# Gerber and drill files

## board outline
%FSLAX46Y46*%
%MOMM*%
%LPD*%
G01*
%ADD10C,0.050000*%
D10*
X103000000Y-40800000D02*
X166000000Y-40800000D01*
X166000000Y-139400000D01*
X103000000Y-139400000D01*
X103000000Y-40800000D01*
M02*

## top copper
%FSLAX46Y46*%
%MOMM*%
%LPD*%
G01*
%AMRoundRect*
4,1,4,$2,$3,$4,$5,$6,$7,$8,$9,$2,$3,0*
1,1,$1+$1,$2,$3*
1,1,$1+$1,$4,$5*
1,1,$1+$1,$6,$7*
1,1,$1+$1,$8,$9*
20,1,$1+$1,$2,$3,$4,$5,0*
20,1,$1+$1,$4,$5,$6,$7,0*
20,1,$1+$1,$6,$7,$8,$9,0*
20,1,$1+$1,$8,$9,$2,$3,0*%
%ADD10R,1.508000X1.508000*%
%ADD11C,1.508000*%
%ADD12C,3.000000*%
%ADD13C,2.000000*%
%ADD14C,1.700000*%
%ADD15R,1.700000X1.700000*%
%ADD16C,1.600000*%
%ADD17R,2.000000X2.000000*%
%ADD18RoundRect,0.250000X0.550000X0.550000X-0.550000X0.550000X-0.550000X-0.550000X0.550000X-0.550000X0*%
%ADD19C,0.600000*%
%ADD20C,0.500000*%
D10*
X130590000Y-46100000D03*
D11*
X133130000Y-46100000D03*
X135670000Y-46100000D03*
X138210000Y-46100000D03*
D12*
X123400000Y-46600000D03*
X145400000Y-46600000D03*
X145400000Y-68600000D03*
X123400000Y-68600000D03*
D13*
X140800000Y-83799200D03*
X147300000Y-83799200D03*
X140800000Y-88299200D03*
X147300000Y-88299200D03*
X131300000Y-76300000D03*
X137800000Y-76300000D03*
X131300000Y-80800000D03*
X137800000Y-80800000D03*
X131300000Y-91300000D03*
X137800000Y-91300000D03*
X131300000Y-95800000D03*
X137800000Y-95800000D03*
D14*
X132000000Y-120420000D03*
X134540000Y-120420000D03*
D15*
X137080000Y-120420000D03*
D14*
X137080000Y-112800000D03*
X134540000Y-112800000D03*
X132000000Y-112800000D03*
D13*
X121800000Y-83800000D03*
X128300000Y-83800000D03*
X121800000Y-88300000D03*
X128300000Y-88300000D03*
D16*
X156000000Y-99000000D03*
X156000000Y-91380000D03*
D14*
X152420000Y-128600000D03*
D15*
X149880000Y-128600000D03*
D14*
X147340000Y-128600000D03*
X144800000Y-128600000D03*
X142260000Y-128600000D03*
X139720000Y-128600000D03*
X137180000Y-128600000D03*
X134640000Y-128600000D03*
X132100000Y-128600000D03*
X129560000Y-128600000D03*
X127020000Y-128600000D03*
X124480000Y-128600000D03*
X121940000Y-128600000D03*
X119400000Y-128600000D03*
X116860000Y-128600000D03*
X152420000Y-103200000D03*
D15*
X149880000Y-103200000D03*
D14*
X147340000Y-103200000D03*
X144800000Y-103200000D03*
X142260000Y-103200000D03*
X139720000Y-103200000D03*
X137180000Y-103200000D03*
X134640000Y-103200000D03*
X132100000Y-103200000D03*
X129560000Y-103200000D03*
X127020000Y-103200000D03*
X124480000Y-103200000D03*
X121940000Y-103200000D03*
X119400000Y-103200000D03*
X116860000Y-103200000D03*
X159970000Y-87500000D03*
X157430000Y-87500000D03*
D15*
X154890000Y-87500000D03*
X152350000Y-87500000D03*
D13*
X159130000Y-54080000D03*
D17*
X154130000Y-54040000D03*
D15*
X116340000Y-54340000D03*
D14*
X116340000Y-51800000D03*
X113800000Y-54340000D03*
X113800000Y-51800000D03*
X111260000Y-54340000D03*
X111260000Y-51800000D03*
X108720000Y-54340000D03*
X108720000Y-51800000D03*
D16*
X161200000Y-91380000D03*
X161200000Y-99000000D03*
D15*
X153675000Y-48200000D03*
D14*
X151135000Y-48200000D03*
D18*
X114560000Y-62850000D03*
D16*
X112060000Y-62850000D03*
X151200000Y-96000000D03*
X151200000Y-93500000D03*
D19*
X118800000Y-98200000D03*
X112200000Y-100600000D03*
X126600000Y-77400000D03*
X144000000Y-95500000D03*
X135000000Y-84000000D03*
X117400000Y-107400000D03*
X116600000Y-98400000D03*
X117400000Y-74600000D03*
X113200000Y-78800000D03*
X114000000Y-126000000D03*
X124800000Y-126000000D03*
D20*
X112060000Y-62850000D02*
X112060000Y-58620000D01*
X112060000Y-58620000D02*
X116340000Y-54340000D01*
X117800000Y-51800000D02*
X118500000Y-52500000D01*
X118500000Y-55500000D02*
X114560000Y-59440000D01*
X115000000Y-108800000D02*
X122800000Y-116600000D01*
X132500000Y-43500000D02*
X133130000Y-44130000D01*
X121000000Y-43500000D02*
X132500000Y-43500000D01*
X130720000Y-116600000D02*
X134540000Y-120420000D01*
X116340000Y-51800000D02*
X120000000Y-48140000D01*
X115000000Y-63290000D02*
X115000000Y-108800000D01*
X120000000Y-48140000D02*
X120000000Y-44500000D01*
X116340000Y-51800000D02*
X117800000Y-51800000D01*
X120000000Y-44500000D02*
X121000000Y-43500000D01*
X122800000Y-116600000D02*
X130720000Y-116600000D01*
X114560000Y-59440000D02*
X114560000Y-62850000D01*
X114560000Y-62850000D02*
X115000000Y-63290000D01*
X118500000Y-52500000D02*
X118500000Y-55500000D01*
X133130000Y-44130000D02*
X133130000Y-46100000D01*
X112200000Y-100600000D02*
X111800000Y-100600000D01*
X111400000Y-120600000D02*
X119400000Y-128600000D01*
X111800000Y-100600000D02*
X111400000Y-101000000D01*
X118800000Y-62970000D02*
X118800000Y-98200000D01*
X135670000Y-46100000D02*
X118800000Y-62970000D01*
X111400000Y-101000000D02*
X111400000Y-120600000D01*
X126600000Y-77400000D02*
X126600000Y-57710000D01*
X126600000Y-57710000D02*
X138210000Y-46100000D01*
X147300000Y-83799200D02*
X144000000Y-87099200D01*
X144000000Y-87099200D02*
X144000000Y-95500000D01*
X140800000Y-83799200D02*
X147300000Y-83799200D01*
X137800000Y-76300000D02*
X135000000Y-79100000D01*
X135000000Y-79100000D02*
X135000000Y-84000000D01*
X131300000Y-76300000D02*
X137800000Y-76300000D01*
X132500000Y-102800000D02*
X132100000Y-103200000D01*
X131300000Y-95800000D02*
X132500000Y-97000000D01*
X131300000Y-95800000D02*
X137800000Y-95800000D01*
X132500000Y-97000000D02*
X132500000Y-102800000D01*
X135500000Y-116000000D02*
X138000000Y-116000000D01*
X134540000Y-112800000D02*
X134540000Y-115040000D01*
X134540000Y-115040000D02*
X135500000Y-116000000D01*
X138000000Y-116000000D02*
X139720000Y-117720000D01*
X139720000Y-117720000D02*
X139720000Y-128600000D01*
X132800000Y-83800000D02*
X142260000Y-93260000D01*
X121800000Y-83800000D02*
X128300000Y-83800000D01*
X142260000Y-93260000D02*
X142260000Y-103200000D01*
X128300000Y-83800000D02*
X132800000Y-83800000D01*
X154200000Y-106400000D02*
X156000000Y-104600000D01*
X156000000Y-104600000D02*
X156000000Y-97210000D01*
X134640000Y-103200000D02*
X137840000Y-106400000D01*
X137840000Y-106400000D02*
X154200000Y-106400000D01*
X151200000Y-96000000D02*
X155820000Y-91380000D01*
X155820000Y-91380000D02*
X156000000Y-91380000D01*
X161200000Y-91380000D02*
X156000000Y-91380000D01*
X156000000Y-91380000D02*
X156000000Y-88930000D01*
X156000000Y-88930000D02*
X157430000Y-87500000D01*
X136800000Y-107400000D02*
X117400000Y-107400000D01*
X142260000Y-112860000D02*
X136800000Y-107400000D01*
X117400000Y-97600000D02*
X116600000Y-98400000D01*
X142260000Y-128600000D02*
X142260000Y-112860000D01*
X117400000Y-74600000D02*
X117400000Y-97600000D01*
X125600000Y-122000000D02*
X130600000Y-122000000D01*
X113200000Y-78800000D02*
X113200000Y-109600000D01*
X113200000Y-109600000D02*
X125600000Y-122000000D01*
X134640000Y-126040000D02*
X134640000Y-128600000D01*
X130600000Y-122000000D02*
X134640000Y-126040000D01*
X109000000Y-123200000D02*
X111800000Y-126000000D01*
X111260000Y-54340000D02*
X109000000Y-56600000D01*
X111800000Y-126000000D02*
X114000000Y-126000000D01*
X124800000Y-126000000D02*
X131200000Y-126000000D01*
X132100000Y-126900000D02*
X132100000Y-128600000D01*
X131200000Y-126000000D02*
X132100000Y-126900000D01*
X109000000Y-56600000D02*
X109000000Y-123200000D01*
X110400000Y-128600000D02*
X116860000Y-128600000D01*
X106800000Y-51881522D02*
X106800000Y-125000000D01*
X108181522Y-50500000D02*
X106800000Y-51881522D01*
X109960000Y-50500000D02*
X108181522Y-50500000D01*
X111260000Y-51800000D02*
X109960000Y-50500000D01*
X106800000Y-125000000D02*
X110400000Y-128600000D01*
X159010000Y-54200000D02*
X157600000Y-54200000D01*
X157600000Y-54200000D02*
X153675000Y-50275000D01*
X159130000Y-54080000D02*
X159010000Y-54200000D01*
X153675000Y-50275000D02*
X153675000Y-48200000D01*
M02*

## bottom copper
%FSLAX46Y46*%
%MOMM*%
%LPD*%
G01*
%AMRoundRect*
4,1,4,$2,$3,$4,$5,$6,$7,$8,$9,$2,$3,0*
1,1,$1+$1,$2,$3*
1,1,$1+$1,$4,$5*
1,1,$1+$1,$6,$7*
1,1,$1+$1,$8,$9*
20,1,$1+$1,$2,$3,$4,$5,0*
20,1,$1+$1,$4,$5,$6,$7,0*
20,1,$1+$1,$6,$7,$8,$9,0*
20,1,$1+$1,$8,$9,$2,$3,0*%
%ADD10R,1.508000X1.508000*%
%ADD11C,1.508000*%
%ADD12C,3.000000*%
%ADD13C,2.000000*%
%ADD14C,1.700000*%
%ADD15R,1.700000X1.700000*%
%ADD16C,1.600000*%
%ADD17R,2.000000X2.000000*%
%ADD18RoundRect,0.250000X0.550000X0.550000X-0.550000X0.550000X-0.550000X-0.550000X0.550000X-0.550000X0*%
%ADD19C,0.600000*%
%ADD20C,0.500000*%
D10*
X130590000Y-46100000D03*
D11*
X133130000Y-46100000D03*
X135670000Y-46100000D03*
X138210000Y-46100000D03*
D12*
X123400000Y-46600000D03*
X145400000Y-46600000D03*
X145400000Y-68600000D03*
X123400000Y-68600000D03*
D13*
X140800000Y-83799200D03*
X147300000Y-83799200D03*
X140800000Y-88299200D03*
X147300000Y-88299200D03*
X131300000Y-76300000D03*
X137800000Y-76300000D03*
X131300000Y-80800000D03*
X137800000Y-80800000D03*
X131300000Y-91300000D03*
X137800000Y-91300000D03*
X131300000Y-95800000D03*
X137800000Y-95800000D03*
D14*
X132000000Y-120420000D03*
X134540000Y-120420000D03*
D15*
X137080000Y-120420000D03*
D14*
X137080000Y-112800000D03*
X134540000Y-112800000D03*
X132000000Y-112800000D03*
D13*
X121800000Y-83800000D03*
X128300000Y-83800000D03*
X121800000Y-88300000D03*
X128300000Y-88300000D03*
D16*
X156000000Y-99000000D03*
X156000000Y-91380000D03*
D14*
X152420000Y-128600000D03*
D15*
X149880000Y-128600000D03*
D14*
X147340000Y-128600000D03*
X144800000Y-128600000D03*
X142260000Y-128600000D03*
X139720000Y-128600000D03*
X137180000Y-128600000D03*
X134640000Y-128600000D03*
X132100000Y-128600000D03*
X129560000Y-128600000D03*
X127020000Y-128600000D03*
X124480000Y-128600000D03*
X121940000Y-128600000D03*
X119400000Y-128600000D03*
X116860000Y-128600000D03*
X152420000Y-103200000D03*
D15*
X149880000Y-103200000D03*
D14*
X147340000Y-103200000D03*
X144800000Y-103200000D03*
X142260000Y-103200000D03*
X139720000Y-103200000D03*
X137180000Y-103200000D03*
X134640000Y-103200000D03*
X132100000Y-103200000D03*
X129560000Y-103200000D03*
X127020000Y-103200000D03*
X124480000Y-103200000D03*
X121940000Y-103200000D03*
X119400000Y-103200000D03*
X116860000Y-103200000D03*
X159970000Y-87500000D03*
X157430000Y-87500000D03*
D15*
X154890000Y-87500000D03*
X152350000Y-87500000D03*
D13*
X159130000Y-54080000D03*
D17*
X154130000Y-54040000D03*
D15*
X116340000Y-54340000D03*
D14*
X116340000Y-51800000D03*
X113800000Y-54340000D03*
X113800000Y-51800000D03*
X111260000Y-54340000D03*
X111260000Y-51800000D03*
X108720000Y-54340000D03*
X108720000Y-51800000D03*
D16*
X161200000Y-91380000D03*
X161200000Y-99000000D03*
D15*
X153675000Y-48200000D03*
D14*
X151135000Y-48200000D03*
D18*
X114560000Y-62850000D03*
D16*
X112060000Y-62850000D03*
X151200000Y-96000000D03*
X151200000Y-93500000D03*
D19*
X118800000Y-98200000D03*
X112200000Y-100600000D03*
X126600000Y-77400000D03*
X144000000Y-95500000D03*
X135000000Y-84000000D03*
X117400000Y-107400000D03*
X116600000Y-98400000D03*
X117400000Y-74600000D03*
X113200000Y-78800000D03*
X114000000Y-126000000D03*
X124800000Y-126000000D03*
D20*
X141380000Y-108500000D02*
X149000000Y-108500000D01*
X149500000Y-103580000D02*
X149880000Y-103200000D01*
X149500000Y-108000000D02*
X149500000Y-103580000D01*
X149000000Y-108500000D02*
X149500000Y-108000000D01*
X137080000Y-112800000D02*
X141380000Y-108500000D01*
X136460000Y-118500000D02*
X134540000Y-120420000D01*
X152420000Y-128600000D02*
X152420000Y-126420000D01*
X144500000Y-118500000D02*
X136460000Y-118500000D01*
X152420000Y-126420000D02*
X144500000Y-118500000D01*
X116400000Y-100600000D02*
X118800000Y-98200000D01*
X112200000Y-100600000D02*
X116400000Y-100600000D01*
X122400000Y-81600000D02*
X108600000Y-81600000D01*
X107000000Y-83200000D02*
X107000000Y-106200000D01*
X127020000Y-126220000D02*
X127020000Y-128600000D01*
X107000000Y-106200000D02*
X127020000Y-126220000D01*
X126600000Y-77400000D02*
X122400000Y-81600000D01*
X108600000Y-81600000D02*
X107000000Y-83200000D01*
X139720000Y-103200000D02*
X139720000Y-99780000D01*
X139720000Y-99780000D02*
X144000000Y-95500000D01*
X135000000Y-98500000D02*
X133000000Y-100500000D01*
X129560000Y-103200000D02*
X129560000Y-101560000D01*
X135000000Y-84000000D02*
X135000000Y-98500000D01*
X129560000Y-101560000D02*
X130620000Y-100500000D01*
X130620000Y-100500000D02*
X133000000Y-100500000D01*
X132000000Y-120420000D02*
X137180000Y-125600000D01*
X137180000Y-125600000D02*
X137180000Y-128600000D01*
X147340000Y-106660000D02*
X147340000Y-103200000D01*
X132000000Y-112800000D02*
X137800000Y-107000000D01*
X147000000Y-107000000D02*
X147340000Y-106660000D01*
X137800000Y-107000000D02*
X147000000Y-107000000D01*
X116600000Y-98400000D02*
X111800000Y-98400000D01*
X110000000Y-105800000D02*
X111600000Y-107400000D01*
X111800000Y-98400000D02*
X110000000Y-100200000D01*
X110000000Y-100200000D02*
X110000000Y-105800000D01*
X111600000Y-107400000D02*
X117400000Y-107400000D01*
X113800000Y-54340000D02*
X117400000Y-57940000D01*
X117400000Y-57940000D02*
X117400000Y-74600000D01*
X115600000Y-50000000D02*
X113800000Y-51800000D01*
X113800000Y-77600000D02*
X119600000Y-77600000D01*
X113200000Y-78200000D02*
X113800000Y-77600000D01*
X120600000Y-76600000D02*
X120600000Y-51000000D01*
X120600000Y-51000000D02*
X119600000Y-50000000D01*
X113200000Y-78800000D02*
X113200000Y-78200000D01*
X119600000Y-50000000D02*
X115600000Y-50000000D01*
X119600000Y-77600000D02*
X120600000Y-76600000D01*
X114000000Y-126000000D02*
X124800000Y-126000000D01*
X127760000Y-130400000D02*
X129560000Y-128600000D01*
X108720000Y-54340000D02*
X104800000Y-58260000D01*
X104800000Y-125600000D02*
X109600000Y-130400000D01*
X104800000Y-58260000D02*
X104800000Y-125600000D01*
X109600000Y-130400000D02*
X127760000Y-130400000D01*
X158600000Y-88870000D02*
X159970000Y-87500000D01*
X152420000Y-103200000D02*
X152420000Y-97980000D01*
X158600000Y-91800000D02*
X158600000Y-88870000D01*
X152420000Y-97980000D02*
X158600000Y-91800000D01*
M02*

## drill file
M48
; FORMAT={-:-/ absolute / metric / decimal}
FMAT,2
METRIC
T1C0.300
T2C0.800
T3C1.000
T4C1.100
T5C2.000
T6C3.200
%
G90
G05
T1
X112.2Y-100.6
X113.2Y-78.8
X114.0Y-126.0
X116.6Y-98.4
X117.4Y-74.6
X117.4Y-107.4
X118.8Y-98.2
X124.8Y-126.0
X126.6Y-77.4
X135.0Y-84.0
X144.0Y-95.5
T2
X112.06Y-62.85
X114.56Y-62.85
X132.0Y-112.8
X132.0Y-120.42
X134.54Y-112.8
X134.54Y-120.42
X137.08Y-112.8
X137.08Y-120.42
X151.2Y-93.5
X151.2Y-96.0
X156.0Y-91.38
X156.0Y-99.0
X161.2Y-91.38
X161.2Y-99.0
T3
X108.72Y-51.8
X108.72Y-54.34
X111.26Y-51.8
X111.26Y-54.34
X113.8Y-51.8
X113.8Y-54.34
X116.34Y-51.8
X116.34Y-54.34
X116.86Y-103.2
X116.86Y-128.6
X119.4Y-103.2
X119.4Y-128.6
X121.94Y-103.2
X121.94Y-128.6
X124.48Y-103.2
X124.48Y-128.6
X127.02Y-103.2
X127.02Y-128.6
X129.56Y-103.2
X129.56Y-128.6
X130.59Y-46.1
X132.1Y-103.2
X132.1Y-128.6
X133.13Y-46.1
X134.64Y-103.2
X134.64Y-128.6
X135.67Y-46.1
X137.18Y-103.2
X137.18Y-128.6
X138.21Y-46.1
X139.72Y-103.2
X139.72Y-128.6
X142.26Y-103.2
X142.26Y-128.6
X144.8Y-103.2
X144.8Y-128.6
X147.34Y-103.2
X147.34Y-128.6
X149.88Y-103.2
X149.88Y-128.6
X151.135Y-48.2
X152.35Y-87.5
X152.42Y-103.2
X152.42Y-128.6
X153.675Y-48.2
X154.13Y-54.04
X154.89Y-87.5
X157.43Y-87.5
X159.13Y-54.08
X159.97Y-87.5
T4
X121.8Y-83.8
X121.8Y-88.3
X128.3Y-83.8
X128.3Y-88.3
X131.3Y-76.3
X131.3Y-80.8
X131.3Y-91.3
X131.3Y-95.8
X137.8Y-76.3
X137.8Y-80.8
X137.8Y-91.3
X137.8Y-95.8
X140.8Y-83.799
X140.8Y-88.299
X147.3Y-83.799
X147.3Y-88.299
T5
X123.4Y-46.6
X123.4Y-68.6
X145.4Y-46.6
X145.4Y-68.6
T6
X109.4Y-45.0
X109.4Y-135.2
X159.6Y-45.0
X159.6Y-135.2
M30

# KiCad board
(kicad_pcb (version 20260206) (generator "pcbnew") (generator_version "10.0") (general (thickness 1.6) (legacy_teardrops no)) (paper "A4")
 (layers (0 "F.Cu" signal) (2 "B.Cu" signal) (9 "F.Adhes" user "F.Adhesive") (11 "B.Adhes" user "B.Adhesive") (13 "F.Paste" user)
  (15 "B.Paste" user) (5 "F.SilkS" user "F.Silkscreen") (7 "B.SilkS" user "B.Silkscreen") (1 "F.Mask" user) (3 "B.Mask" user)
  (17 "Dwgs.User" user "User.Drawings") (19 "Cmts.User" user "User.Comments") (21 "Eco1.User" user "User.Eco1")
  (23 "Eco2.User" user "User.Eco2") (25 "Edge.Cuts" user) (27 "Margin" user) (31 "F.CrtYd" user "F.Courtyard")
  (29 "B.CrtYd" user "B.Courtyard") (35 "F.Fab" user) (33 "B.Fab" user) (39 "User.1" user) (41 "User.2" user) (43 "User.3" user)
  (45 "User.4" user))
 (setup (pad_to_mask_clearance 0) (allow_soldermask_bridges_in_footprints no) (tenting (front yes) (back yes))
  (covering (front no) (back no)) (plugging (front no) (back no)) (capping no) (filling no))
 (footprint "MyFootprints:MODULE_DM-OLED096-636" (layer "F.Cu") (at 134.4 57.6)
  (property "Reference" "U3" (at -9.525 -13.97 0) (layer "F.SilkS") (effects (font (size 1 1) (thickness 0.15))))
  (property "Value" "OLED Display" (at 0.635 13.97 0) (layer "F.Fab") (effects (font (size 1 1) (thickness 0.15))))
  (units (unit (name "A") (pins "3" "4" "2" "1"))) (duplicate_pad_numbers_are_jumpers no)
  (pad "1" thru_hole rect (at -3.81 -11.5) (size 1.508 1.508) (drill 1) (layers "*.Cu" "*.Mask") (remove_unused_layers no) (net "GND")
   (solder_mask_margin 0.102))
  (pad "2" thru_hole circle (at -1.27 -11.5) (size 1.508 1.508) (drill 1) (layers "*.Cu" "*.Mask") (remove_unused_layers no) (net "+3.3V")
   (solder_mask_margin 0.102))
  (pad "3" thru_hole circle (at 1.27 -11.5) (size 1.508 1.508) (drill 1) (layers "*.Cu" "*.Mask") (remove_unused_layers no) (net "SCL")
   (solder_mask_margin 0.102))
  (pad "4" thru_hole circle (at 3.81 -11.5) (size 1.508 1.508) (drill 1) (layers "*.Cu" "*.Mask") (remove_unused_layers no) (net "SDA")
   (solder_mask_margin 0.102))
  (pad "S1" thru_hole circle (at -11 -11) (size 3 3) (drill 2) (layers "*.Cu" "*.Mask") (remove_unused_layers no) (solder_mask_margin 0.102))
  (pad "S2" thru_hole circle (at 11 -11) (size 3 3) (drill 2) (layers "*.Cu" "*.Mask") (remove_unused_layers no) (solder_mask_margin 0.102))
  (pad "S3" thru_hole circle (at 11 11) (size 3 3) (drill 2) (layers "*.Cu" "*.Mask") (remove_unused_layers no) (solder_mask_margin 0.102))
  (pad "S4" thru_hole circle (at -11 11) (size 3 3) (drill 2) (layers "*.Cu" "*.Mask") (remove_unused_layers no) (solder_mask_margin 0.102)))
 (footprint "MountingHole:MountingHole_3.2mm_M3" (layer "F.Cu") (at 159.6 45)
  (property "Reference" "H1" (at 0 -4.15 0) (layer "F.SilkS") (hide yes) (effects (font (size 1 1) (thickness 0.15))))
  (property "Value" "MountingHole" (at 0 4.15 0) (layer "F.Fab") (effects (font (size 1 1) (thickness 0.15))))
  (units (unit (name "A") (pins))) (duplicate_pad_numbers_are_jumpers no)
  (pad "" np_thru_hole circle (at 0 0) (size 3.2 3.2) (drill 3.2) (layers "*.Cu" "*.Mask")))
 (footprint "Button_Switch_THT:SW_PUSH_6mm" (layer "F.Cu") (at 140.8 83.7992)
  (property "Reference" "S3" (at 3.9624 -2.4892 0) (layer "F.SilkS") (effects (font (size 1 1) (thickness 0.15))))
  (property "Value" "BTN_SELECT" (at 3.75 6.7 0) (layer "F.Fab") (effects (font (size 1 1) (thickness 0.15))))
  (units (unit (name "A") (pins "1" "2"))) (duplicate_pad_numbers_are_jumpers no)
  (pad "1" thru_hole circle (at 0 0 90) (size 2 2) (drill 1.1) (layers "*.Cu" "*.Mask") (remove_unused_layers no) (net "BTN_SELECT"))
  (pad "1" thru_hole circle (at 6.5 0 90) (size 2 2) (drill 1.1) (layers "*.Cu" "*.Mask") (remove_unused_layers no) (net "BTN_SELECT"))
  (pad "2" thru_hole circle (at 0 4.5 90) (size 2 2) (drill 1.1) (layers "*.Cu" "*.Mask") (remove_unused_layers no) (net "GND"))
  (pad "2" thru_hole circle (at 6.5 4.5 90) (size 2 2) (drill 1.1) (layers "*.Cu" "*.Mask") (remove_unused_layers no) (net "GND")))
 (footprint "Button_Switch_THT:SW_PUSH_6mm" (layer "F.Cu") (at 131.3 76.3)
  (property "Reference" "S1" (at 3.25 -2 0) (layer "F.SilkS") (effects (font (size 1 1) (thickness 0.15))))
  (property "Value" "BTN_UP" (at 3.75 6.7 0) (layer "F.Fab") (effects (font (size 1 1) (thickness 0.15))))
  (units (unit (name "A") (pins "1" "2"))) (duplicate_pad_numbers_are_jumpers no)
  (pad "1" thru_hole circle (at 0 0 90) (size 2 2) (drill 1.1) (layers "*.Cu" "*.Mask") (remove_unused_layers no) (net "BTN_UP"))
  (pad "1" thru_hole circle (at 6.5 0 90) (size 2 2) (drill 1.1) (layers "*.Cu" "*.Mask") (remove_unused_layers no) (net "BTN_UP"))
  (pad "2" thru_hole circle (at 0 4.5 90) (size 2 2) (drill 1.1) (layers "*.Cu" "*.Mask") (remove_unused_layers no) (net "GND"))
  (pad "2" thru_hole circle (at 6.5 4.5 90) (size 2 2) (drill 1.1) (layers "*.Cu" "*.Mask") (remove_unused_layers no) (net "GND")))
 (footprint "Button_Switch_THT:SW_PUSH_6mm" (layer "F.Cu") (at 131.3 91.3)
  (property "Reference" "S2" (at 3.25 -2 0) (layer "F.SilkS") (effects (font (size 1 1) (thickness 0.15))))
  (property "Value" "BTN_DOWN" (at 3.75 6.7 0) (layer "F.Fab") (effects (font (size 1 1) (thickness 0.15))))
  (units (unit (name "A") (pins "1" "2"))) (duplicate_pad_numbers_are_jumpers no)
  (pad "1" thru_hole circle (at 0 0 90) (size 2 2) (drill 1.1) (layers "*.Cu" "*.Mask") (remove_unused_layers no) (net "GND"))
  (pad "1" thru_hole circle (at 6.5 0 90) (size 2 2) (drill 1.1) (layers "*.Cu" "*.Mask") (remove_unused_layers no) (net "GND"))
  (pad "2" thru_hole circle (at 0 4.5 90) (size 2 2) (drill 1.1) (layers "*.Cu" "*.Mask") (remove_unused_layers no) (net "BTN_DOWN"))
  (pad "2" thru_hole circle (at 6.5 4.5 90) (size 2 2) (drill 1.1) (layers "*.Cu" "*.Mask") (remove_unused_layers no) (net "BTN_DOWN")))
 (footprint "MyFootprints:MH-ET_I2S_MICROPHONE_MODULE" (layer "F.Cu") (at 134.54 115.34)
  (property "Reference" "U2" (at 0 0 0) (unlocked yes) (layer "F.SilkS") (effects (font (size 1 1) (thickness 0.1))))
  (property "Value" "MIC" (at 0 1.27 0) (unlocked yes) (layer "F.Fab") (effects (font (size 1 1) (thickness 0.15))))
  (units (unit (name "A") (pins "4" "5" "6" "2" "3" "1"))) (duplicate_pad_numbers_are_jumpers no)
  (pad "1" thru_hole circle (at -2.54 5.08) (size 1.7 1.7) (drill 0.8) (layers "*.Cu" "*.Mask") (remove_unused_layers no) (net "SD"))
  (pad "2" thru_hole circle (at 0 5.08) (size 1.7 1.7) (drill 0.8) (layers "*.Cu" "*.Mask") (remove_unused_layers no) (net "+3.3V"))
  (pad "3" thru_hole rect (at 2.54 5.08) (size 1.7 1.7) (drill 0.8) (layers "*.Cu" "*.Mask") (remove_unused_layers no) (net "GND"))
  (pad "4" thru_hole circle (at 2.54 -2.54) (size 1.7 1.7) (drill 0.8) (layers "*.Cu" "*.Mask") (remove_unused_layers no) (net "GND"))
  (pad "5" thru_hole circle (at 0 -2.54) (size 1.7 1.7) (drill 0.8) (layers "*.Cu" "*.Mask") (remove_unused_layers no) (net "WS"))
  (pad "6" thru_hole circle (at -2.54 -2.54) (size 1.7 1.7) (drill 0.8) (layers "*.Cu" "*.Mask") (remove_unused_layers no) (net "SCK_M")))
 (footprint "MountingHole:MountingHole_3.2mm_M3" (layer "F.Cu") (at 159.6 135.2)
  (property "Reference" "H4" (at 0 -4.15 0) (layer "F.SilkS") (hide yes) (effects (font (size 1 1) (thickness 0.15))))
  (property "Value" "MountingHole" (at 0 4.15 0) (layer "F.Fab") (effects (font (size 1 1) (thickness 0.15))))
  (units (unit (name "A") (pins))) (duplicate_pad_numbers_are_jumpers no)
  (pad "" np_thru_hole circle (at 0 0) (size 3.2 3.2) (drill 3.2) (layers "*.Cu" "*.Mask")))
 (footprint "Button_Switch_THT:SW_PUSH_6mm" (layer "F.Cu") (at 121.8 83.8)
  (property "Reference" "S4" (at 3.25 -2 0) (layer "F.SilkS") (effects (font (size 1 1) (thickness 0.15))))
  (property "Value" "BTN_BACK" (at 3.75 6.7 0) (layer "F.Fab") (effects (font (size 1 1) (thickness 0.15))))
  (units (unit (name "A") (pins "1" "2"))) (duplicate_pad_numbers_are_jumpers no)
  (pad "1" thru_hole circle (at 0 0 90) (size 2 2) (drill 1.1) (layers "*.Cu" "*.Mask") (remove_unused_layers no) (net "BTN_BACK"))
  (pad "1" thru_hole circle (at 6.5 0 90) (size 2 2) (drill 1.1) (layers "*.Cu" "*.Mask") (remove_unused_layers no) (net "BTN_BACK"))
  (pad "2" thru_hole circle (at 0 4.5 90) (size 2 2) (drill 1.1) (layers "*.Cu" "*.Mask") (remove_unused_layers no) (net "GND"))
  (pad "2" thru_hole circle (at 6.5 4.5 90) (size 2 2) (drill 1.1) (layers "*.Cu" "*.Mask") (remove_unused_layers no) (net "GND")))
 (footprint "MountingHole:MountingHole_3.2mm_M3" (layer "F.Cu") (at 109.4 135.2)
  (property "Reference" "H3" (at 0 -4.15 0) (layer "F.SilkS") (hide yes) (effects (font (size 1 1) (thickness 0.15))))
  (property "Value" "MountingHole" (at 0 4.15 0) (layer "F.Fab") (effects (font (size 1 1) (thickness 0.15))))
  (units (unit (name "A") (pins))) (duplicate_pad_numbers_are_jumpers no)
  (pad "" np_thru_hole circle (at 0 0) (size 3.2 3.2) (drill 3.2) (layers "*.Cu" "*.Mask")))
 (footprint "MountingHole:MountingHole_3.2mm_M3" (layer "F.Cu") (at 109.4 45)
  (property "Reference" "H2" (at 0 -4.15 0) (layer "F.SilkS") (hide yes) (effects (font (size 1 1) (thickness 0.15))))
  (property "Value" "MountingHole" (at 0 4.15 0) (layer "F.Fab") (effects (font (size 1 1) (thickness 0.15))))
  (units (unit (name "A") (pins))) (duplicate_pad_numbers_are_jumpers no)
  (pad "" np_thru_hole circle (at 0 0) (size 3.2 3.2) (drill 3.2) (layers "*.Cu" "*.Mask")))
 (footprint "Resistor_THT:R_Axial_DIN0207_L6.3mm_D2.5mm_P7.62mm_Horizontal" (layer "B.Cu") (at 156 99 90)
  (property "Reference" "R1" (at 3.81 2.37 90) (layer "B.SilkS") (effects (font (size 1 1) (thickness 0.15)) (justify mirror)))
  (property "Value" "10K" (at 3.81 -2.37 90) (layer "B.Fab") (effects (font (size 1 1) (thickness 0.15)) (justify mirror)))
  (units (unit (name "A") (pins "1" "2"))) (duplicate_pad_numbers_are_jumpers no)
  (pad "1" thru_hole circle (at 0 0 90) (size 1.6 1.6) (drill 0.8) (layers "*.Cu" "*.Mask") (remove_unused_layers no) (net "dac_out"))
  (pad "2" thru_hole circle (at 7.62 0 90) (size 1.6 1.6) (drill 0.8) (layers "*.Cu" "*.Mask") (remove_unused_layers no) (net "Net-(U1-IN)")))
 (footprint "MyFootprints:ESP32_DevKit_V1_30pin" (layer "B.Cu") (at 152.42 128.6 90)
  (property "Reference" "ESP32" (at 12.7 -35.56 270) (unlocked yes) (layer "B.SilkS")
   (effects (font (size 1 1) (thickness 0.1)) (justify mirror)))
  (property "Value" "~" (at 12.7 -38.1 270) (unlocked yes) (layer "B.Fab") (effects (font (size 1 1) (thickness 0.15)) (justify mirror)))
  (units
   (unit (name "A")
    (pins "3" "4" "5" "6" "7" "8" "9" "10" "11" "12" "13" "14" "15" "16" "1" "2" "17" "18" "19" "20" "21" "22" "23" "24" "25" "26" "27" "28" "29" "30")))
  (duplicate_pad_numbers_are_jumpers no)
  (pad "1" thru_hole circle (at 0 0 90) (size 1.7 1.7) (drill 1) (layers "*.Cu" "*.Mask") (remove_unused_layers no) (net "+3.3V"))
  (pad "2" thru_hole rect (at 0 -2.54 90) (size 1.7 1.7) (drill 1) (layers "*.Cu" "*.Mask") (remove_unused_layers no) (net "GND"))
  (pad "3" thru_hole circle (at 0 -5.08 90) (size 1.7 1.7) (drill 1) (layers "*.Cu" "*.Mask") (remove_unused_layers no)
   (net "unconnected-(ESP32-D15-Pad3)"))
  (pad "4" thru_hole circle (at 0 -7.62 90) (size 1.7 1.7) (drill 1) (layers "*.Cu" "*.Mask") (remove_unused_layers no)
   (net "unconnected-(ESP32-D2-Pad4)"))
  (pad "5" thru_hole circle (at 0 -10.16 90) (size 1.7 1.7) (drill 1) (layers "*.Cu" "*.Mask") (remove_unused_layers no) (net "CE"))
  (pad "6" thru_hole circle (at 0 -12.7 90) (size 1.7 1.7) (drill 1) (layers "*.Cu" "*.Mask") (remove_unused_layers no) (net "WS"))
  (pad "7" thru_hole circle (at 0 -15.24 90) (size 1.7 1.7) (drill 1) (layers "*.Cu" "*.Mask") (remove_unused_layers no) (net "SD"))
  (pad "8" thru_hole circle (at 0 -17.78 90) (size 1.7 1.7) (drill 1) (layers "*.Cu" "*.Mask") (remove_unused_layers no) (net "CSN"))
  (pad "9" thru_hole circle (at 0 -20.32 90) (size 1.7 1.7) (drill 1) (layers "*.Cu" "*.Mask") (remove_unused_layers no) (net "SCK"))
  (pad "10" thru_hole circle (at 0 -22.86 90) (size 1.7 1.7) (drill 1) (layers "*.Cu" "*.Mask") (remove_unused_layers no) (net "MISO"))
  (pad "11" thru_hole circle (at 0 -25.4 90) (size 1.7 1.7) (drill 1) (layers "*.Cu" "*.Mask") (remove_unused_layers no) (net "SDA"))
  (pad "12" thru_hole circle (at 0 -27.94 90) (size 1.7 1.7) (drill 1) (layers "*.Cu" "*.Mask") (remove_unused_layers no)
   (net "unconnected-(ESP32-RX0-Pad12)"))
  (pad "13" thru_hole circle (at 0 -30.48 90) (size 1.7 1.7) (drill 1) (layers "*.Cu" "*.Mask") (remove_unused_layers no)
   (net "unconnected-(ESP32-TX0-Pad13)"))
  (pad "14" thru_hole circle (at 0 -33.02 90) (size 1.7 1.7) (drill 1) (layers "*.Cu" "*.Mask") (remove_unused_layers no) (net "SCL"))
  (pad "15" thru_hole circle (at 0 -35.56 90) (size 1.7 1.7) (drill 1) (layers "*.Cu" "*.Mask") (remove_unused_layers no) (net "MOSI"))
  (pad "16" thru_hole circle (at 25.4 0 90) (size 1.7 1.7) (drill 1) (layers "*.Cu" "*.Mask") (remove_unused_layers no) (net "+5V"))
  (pad "17" thru_hole rect (at 25.4 -2.54 90) (size 1.7 1.7) (drill 1) (layers "*.Cu" "*.Mask") (remove_unused_layers no) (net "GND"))
  (pad "18" thru_hole circle (at 25.4 -5.08 90) (size 1.7 1.7) (drill 1) (layers "*.Cu" "*.Mask") (remove_unused_layers no) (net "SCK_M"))
  (pad "19" thru_hole circle (at 25.4 -7.62 90) (size 1.7 1.7) (drill 1) (layers "*.Cu" "*.Mask") (remove_unused_layers no)
   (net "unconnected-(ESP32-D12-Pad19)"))
  (pad "20" thru_hole circle (at 25.4 -10.16 90) (size 1.7 1.7) (drill 1) (layers "*.Cu" "*.Mask") (remove_unused_layers no)
   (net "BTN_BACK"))
  (pad "21" thru_hole circle (at 25.4 -12.7 90) (size 1.7 1.7) (drill 1) (layers "*.Cu" "*.Mask") (remove_unused_layers no)
   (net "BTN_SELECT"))
  (pad "22" thru_hole circle (at 25.4 -15.24 90) (size 1.7 1.7) (drill 1) (layers "*.Cu" "*.Mask") (remove_unused_layers no)
   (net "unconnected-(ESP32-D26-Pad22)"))
  (pad "23" thru_hole circle (at 25.4 -17.78 90) (size 1.7 1.7) (drill 1) (layers "*.Cu" "*.Mask") (remove_unused_layers no) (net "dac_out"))
  (pad "24" thru_hole circle (at 25.4 -20.32 90) (size 1.7 1.7) (drill 1) (layers "*.Cu" "*.Mask") (remove_unused_layers no)
   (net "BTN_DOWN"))
  (pad "25" thru_hole circle (at 25.4 -22.86 90) (size 1.7 1.7) (drill 1) (layers "*.Cu" "*.Mask") (remove_unused_layers no) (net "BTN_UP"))
  (pad "26" thru_hole circle (at 25.4 -25.4 90) (size 1.7 1.7) (drill 1) (layers "*.Cu" "*.Mask") (remove_unused_layers no)
   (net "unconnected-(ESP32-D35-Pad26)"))
  (pad "27" thru_hole circle (at 25.4 -27.94 90) (size 1.7 1.7) (drill 1) (layers "*.Cu" "*.Mask") (remove_unused_layers no)
   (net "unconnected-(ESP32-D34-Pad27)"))
  (pad "28" thru_hole circle (at 25.4 -30.48 90) (size 1.7 1.7) (drill 1) (layers "*.Cu" "*.Mask") (remove_unused_layers no)
   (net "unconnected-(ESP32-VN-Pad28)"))
  (pad "29" thru_hole circle (at 25.4 -33.02 90) (size 1.7 1.7) (drill 1) (layers "*.Cu" "*.Mask") (remove_unused_layers no)
   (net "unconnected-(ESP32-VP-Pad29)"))
  (pad "30" thru_hole circle (at 25.4 -35.56 90) (size 1.7 1.7) (drill 1) (layers "*.Cu" "*.Mask") (remove_unused_layers no)
   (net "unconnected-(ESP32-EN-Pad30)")))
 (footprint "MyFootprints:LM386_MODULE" (layer "B.Cu") (at 160.48 87.5 90)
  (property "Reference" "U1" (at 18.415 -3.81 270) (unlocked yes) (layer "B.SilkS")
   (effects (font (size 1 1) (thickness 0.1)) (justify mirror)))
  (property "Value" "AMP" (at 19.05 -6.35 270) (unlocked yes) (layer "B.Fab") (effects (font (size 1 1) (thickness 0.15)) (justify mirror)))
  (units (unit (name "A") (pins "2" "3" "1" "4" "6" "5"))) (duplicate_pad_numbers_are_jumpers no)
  (pad "1" thru_hole circle (at 0 -0.51 90) (size 1.7 1.7) (drill 1) (layers "*.Cu" "*.Mask") (remove_unused_layers no) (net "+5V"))
  (pad "2" thru_hole circle (at 0 -3.05 90) (size 1.7 1.7) (drill 1) (layers "*.Cu" "*.Mask") (remove_unused_layers no) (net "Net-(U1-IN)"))
  (pad "3" thru_hole rect (at 0 -5.59 90) (size 1.7 1.7) (drill 1) (layers "*.Cu" "*.Mask") (remove_unused_layers no) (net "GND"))
  (pad "4" thru_hole rect (at 0 -8.13 90) (size 1.7 1.7) (drill 1) (layers "*.Cu" "*.Mask") (remove_unused_layers no) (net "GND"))
  (pad "5" thru_hole circle (at 33.42 -1.35 90) (size 2 2) (drill 1) (layers "*.Cu" "*.Mask") (remove_unused_layers no)
   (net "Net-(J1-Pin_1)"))
  (pad "6" thru_hole rect (at 33.46 -6.35 90) (size 2 2) (drill 1) (layers "*.Cu" "*.Mask") (remove_unused_layers no) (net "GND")))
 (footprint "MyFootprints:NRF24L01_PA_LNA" (layer "B.Cu") (at 108.73 54.3 180)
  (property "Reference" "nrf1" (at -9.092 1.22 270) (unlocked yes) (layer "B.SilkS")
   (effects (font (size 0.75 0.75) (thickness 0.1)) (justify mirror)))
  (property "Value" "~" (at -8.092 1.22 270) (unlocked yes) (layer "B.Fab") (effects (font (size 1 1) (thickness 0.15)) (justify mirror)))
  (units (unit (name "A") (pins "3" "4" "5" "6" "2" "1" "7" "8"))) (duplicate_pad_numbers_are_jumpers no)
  (pad "1" thru_hole rect (at -7.61 -0.04 270) (size 1.7 1.7) (drill 1) (layers "*.Cu" "*.Mask") (remove_unused_layers no) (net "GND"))
  (pad "2" thru_hole circle (at -7.61 2.5 270) (size 1.7 1.7) (drill 1) (layers "*.Cu" "*.Mask") (remove_unused_layers no) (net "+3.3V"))
  (pad "3" thru_hole circle (at -5.07 -0.04 270) (size 1.7 1.7) (drill 1) (layers "*.Cu" "*.Mask") (remove_unused_layers no) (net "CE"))
  (pad "4" thru_hole circle (at -5.07 2.5 270) (size 1.7 1.7) (drill 1) (layers "*.Cu" "*.Mask") (remove_unused_layers no) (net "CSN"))
  (pad "5" thru_hole circle (at -2.53 -0.04 270) (size 1.7 1.7) (drill 1) (layers "*.Cu" "*.Mask") (remove_unused_layers no) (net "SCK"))
  (pad "6" thru_hole circle (at -2.53 2.5 270) (size 1.7 1.7) (drill 1) (layers "*.Cu" "*.Mask") (remove_unused_layers no) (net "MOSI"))
  (pad "7" thru_hole circle (at 0.01 -0.04 270) (size 1.7 1.7) (drill 1) (layers "*.Cu" "*.Mask") (remove_unused_layers no) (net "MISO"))
  (pad "8" thru_hole circle (at 0.01 2.5 270) (size 1.7 1.7) (drill 1) (layers "*.Cu" "*.Mask") (remove_unused_layers no)
   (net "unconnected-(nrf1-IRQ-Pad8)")))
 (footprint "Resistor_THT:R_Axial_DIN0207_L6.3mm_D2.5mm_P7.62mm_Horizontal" (layer "B.Cu") (at 161.2 91.38 -90)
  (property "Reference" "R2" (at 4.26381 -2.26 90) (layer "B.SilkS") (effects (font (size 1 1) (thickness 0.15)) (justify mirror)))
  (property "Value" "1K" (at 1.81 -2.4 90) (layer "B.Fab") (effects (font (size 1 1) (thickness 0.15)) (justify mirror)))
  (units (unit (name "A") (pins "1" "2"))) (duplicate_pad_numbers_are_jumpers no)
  (pad "1" thru_hole circle (at 0 0 270) (size 1.6 1.6) (drill 0.8) (layers "*.Cu" "*.Mask") (remove_unused_layers no) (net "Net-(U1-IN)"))
  (pad "2" thru_hole circle (at 7.62 0 270) (size 1.6 1.6) (drill 0.8) (layers "*.Cu" "*.Mask") (remove_unused_layers no) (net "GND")))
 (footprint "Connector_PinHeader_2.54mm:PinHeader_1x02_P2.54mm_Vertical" (layer "B.Cu") (at 153.675 48.2 90)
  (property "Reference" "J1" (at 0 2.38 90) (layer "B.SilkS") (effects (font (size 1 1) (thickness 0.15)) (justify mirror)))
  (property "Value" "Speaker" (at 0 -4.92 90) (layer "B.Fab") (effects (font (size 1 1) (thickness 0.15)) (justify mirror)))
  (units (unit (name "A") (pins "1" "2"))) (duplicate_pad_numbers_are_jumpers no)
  (pad "1" thru_hole rect (at 0 0 90) (size 1.7 1.7) (drill 1) (layers "*.Cu" "*.Mask") (remove_unused_layers no) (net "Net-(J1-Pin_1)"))
  (pad "2" thru_hole circle (at 0 -2.54 90) (size 1.7 1.7) (drill 1) (layers "*.Cu" "*.Mask") (remove_unused_layers no) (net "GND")))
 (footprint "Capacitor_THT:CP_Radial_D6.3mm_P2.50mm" (layer "B.Cu") (at 114.56 62.85 180)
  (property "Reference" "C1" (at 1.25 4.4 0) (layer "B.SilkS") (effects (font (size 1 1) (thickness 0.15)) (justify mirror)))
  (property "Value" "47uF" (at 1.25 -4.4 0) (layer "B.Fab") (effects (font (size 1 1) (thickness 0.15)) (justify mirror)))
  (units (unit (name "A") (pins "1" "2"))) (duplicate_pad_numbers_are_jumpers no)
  (pad "1" thru_hole roundrect (at 0 0 180) (size 1.6 1.6) (drill 0.8) (layers "*.Cu" "*.Mask") (remove_unused_layers no)
   (roundrect_rratio 0.15625) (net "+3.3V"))
  (pad "2" thru_hole circle (at 2.5 0 180) (size 1.6 1.6) (drill 0.8) (layers "*.Cu" "*.Mask") (remove_unused_layers no) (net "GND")))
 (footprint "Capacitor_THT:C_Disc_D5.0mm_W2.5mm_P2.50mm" (layer "B.Cu") (at 151.2 96 90)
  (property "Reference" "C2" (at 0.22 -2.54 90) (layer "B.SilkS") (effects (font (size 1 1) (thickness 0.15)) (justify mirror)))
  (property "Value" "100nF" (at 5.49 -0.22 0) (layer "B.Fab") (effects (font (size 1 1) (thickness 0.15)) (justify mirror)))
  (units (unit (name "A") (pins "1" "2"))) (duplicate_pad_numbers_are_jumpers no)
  (pad "1" thru_hole circle (at 0 0 90) (size 1.6 1.6) (drill 0.8) (layers "*.Cu" "*.Mask") (remove_unused_layers no) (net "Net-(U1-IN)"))
  (pad "2" thru_hole circle (at 2.5 0 90) (size 1.6 1.6) (drill 0.8) (layers "*.Cu" "*.Mask") (remove_unused_layers no) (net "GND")))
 (gr_rect (start 103 40.8) (end 166 139.4) (stroke (width 0.05) (type solid)) (fill no) (layer "Edge.Cuts"))
 (segment (start 112.06 62.85) (end 112.06 58.62) (width 0.5) (layer "F.Cu") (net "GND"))
 (segment (start 112.06 58.62) (end 116.34 54.34) (width 0.5) (layer "F.Cu") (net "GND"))
 (segment (start 141.38 108.5) (end 149 108.5) (width 0.5) (layer "B.Cu") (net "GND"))
 (segment (start 149.5 103.58) (end 149.88 103.2) (width 0.5) (layer "B.Cu") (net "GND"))
 (segment (start 149.5 108) (end 149.5 103.58) (width 0.5) (layer "B.Cu") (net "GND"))
 (segment (start 149 108.5) (end 149.5 108) (width 0.5) (layer "B.Cu") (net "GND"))
 (segment (start 137.08 112.8) (end 141.38 108.5) (width 0.5) (layer "B.Cu") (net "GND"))
 (segment (start 117.8 51.8) (end 118.5 52.5) (width 0.5) (layer "F.Cu") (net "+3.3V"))
 (segment (start 118.5 55.5) (end 114.56 59.44) (width 0.5) (layer "F.Cu") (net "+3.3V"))
 (segment (start 115 108.8) (end 122.8 116.6) (width 0.5) (layer "F.Cu") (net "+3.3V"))
 (segment (start 132.5 43.5) (end 133.13 44.13) (width 0.5) (layer "F.Cu") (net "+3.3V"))
 (segment (start 121 43.5) (end 132.5 43.5) (width 0.5) (layer "F.Cu") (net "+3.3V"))
 (segment (start 130.72 116.6) (end 134.54 120.42) (width 0.5) (layer "F.Cu") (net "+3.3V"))
 (segment (start 116.34 51.8) (end 120 48.14) (width 0.5) (layer "F.Cu") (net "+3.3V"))
 (segment (start 115 63.29) (end 115 108.8) (width 0.5) (layer "F.Cu") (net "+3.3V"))
 (segment (start 120 48.14) (end 120 44.5) (width 0.5) (layer "F.Cu") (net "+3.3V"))
 (segment (start 116.34 51.8) (end 117.8 51.8) (width 0.5) (layer "F.Cu") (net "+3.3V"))
 (segment (start 120 44.5) (end 121 43.5) (width 0.5) (layer "F.Cu") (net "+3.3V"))
 (segment (start 122.8 116.6) (end 130.72 116.6) (width 0.5) (layer "F.Cu") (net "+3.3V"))
 (segment (start 114.56 59.44) (end 114.56 62.85) (width 0.5) (layer "F.Cu") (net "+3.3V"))
 (segment (start 114.56 62.85) (end 115 63.29) (width 0.5) (layer "F.Cu") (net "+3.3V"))
 (segment (start 118.5 52.5) (end 118.5 55.5) (width 0.5) (layer "F.Cu") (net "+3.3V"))
 (segment (start 133.13 44.13) (end 133.13 46.1) (width 0.5) (layer "F.Cu") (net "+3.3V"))
 (segment (start 136.46 118.5) (end 134.54 120.42) (width 0.5) (layer "B.Cu") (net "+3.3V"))
 (segment (start 152.42 128.6) (end 152.42 126.42) (width 0.5) (layer "B.Cu") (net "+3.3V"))
 (segment (start 144.5 118.5) (end 136.46 118.5) (width 0.5) (layer "B.Cu") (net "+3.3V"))
 (segment (start 152.42 126.42) (end 144.5 118.5) (width 0.5) (layer "B.Cu") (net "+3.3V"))
 (segment (start 112.2 100.6) (end 111.8 100.6) (width 0.5) (layer "F.Cu") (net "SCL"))
 (segment (start 111.4 120.6) (end 119.4 128.6) (width 0.5) (layer "F.Cu") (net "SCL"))
 (segment (start 111.8 100.6) (end 111.4 101) (width 0.5) (layer "F.Cu") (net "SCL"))
 (segment (start 118.8 62.97) (end 118.8 98.2) (width 0.5) (layer "F.Cu") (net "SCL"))
 (segment (start 135.67 46.1) (end 118.8 62.97) (width 0.5) (layer "F.Cu") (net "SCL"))
 (segment (start 111.4 101) (end 111.4 120.6) (width 0.5) (layer "F.Cu") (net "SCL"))
 (via (at 118.8 98.2) (size 0.6) (drill 0.3) (layers "F.Cu" "B.Cu") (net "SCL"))
 (via (at 112.2 100.6) (size 0.6) (drill 0.3) (layers "F.Cu" "B.Cu") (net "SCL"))
 (segment (start 116.4 100.6) (end 118.8 98.2) (width 0.5) (layer "B.Cu") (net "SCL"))
 (segment (start 112.2 100.6) (end 116.4 100.6) (width 0.5) (layer "B.Cu") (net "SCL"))
 (segment (start 126.6 77.4) (end 126.6 57.71) (width 0.5) (layer "F.Cu") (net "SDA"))
 (segment (start 126.6 57.71) (end 138.21 46.1) (width 0.5) (layer "F.Cu") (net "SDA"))
 (via (at 126.6 77.4) (size 0.6) (drill 0.3) (layers "F.Cu" "B.Cu") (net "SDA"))
 (segment (start 122.4 81.6) (end 108.6 81.6) (width 0.5) (layer "B.Cu") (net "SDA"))
 (segment (start 107 83.2) (end 107 106.2) (width 0.5) (layer "B.Cu") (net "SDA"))
 (segment (start 127.02 126.22) (end 127.02 128.6) (width 0.5) (layer "B.Cu") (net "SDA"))
 (segment (start 107 106.2) (end 127.02 126.22) (width 0.5) (layer "B.Cu") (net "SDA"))
 (segment (start 126.6 77.4) (end 122.4 81.6) (width 0.5) (layer "B.Cu") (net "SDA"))
 (segment (start 108.6 81.6) (end 107 83.2) (width 0.5) (layer "B.Cu") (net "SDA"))
 (segment (start 147.3 83.7992) (end 144 87.0992) (width 0.5) (layer "F.Cu") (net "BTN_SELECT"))
 (segment (start 144 87.0992) (end 144 95.5) (width 0.5) (layer "F.Cu") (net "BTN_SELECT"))
 (segment (start 140.8 83.7992) (end 147.3 83.7992) (width 0.5) (layer "F.Cu") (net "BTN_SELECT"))
 (via (at 144 95.5) (size 0.6) (drill 0.3) (layers "F.Cu" "B.Cu") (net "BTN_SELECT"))
 (segment (start 139.72 103.2) (end 139.72 99.78) (width 0.5) (layer "B.Cu") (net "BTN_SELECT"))
 (segment (start 139.72 99.78) (end 144 95.5) (width 0.5) (layer "B.Cu") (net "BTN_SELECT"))
 (segment (start 137.8 76.3) (end 135 79.1) (width 0.5) (layer "F.Cu") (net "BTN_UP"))
 (segment (start 135 79.1) (end 135 84) (width 0.5) (layer "F.Cu") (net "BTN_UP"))
 (segment (start 131.3 76.3) (end 137.8 76.3) (width 0.5) (layer "F.Cu") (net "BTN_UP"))
 (via (at 135 84) (size 0.6) (drill 0.3) (layers "F.Cu" "B.Cu") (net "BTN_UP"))
 (segment (start 135 98.5) (end 133 100.5) (width 0.5) (layer "B.Cu") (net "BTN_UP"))
 (segment (start 129.56 103.2) (end 129.56 101.56) (width 0.5) (layer "B.Cu") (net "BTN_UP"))
 (segment (start 135 84) (end 135 98.5) (width 0.5) (layer "B.Cu") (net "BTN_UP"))
 (segment (start 129.56 101.56) (end 130.62 100.5) (width 0.5) (layer "B.Cu") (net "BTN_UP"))
 (segment (start 130.62 100.5) (end 133 100.5) (width 0.5) (layer "B.Cu") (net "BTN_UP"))
 (segment (start 132.5 102.8) (end 132.1 103.2) (width 0.5) (layer "F.Cu") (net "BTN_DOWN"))
 (segment (start 131.3 95.8) (end 132.5 97) (width 0.5) (layer "F.Cu") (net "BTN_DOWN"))
 (segment (start 131.3 95.8) (end 137.8 95.8) (width 0.5) (layer "F.Cu") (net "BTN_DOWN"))
 (segment (start 132.5 97) (end 132.5 102.8) (width 0.5) (layer "F.Cu") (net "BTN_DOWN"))
 (segment (start 132 120.42) (end 137.18 125.6) (width 0.5) (layer "B.Cu") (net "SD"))
 (segment (start 137.18 125.6) (end 137.18 128.6) (width 0.5) (layer "B.Cu") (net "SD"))
 (segment (start 135.5 116) (end 138 116) (width 0.5) (layer "F.Cu") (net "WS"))
 (segment (start 134.54 112.8) (end 134.54 115.04) (width 0.5) (layer "F.Cu") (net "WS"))
 (segment (start 134.54 115.04) (end 135.5 116) (width 0.5) (layer "F.Cu") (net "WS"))
 (segment (start 138 116) (end 139.72 117.72) (width 0.5) (layer "F.Cu") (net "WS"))
 (segment (start 139.72 117.72) (end 139.72 128.6) (width 0.5) (layer "F.Cu") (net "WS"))
 (segment (start 147.34 106.66) (end 147.34 103.2) (width 0.5) (layer "B.Cu") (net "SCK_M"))
 (segment (start 132 112.8) (end 137.8 107) (width 0.5) (layer "B.Cu") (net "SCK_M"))
 (segment (start 147 107) (end 147.34 106.66) (width 0.5) (layer "B.Cu") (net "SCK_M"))
 (segment (start 137.8 107) (end 147 107) (width 0.5) (layer "B.Cu") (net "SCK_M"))
 (segment (start 132.8 83.8) (end 142.26 93.26) (width 0.5) (layer "F.Cu") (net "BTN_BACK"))
 (segment (start 121.8 83.8) (end 128.3 83.8) (width 0.5) (layer "F.Cu") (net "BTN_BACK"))
 (segment (start 142.26 93.26) (end 142.26 103.2) (width 0.5) (layer "F.Cu") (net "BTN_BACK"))
 (segment (start 128.3 83.8) (end 132.8 83.8) (width 0.5) (layer "F.Cu") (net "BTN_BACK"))
 (segment (start 154.2 106.4) (end 156 104.6) (width 0.5) (layer "F.Cu") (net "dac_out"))
 (segment (start 156 104.6) (end 156 97.21) (width 0.5) (layer "F.Cu") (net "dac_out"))
 (segment (start 134.64 103.2) (end 137.84 106.4) (width 0.5) (layer "F.Cu") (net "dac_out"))
 (segment (start 137.84 106.4) (end 154.2 106.4) (width 0.5) (layer "F.Cu") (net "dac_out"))
 (segment (start 151.2 96) (end 155.82 91.38) (width 0.5) (layer "F.Cu") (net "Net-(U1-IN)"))
 (segment (start 155.82 91.38) (end 156 91.38) (width 0.5) (layer "F.Cu") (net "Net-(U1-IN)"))
 (segment (start 161.2 91.38) (end 156 91.38) (width 0.5) (layer "F.Cu") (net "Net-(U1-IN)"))
 (segment (start 156 91.38) (end 156 88.93) (width 0.5) (layer "F.Cu") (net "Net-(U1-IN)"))
 (segment (start 156 88.93) (end 157.43 87.5) (width 0.5) (layer "F.Cu") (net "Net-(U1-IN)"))
 (segment (start 136.8 107.4) (end 117.4 107.4) (width 0.5) (layer "F.Cu") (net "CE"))
 (segment (start 142.26 112.86) (end 136.8 107.4) (width 0.5) (layer "F.Cu") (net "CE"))
 (segment (start 117.4 97.6) (end 116.6 98.4) (width 0.5) (layer "F.Cu") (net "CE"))
 (segment (start 142.26 128.6) (end 142.26 112.86) (width 0.5) (layer "F.Cu") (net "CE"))
 (segment (start 117.4 74.6) (end 117.4 97.6) (width 0.5) (layer "F.Cu") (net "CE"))
 (via (at 117.4 107.4) (size 0.6) (drill 0.3) (layers "F.Cu" "B.Cu") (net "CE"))
 (via (at 116.6 98.4) (size 0.6) (drill 0.3) (layers "F.Cu" "B.Cu") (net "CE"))
 (via (at 117.4 74.6) (size 0.6) (drill 0.3) (layers "F.Cu" "B.Cu") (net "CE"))
 (segment (start 116.6 98.4) (end 111.8 98.4) (width 0.5) (layer "B.Cu") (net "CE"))
 (segment (start 110 105.8) (end 111.6 107.4) (width 0.5) (layer "B.Cu") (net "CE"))
 (segment (start 111.8 98.4) (end 110 100.2) (width 0.5) (layer "B.Cu") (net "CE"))
 (segment (start 110 100.2) (end 110 105.8) (width 0.5) (layer "B.Cu") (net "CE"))
 (segment (start 111.6 107.4) (end 117.4 107.4) (width 0.5) (layer "B.Cu") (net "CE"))
 (segment (start 113.8 54.34) (end 117.4 57.94) (width 0.5) (layer "B.Cu") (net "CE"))
 (segment (start 117.4 57.94) (end 117.4 74.6) (width 0.5) (layer "B.Cu") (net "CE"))
 (segment (start 125.6 122) (end 130.6 122) (width 0.5) (layer "F.Cu") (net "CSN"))
 (segment (start 113.2 78.8) (end 113.2 109.6) (width 0.5) (layer "F.Cu") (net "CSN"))
 (segment (start 113.2 109.6) (end 125.6 122) (width 0.5) (layer "F.Cu") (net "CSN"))
 (segment (start 134.64 126.04) (end 134.64 128.6) (width 0.5) (layer "F.Cu") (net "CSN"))
 (segment (start 130.6 122) (end 134.64 126.04) (width 0.5) (layer "F.Cu") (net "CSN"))
 (via (at 113.2 78.8) (size 0.6) (drill 0.3) (layers "F.Cu" "B.Cu") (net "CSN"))
 (segment (start 115.6 50) (end 113.8 51.8) (width 0.5) (layer "B.Cu") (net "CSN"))
 (segment (start 113.8 77.6) (end 119.6 77.6) (width 0.5) (layer "B.Cu") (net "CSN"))
 (segment (start 113.2 78.2) (end 113.8 77.6) (width 0.5) (layer "B.Cu") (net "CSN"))
 (segment (start 120.6 76.6) (end 120.6 51) (width 0.5) (layer "B.Cu") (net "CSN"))
 (segment (start 120.6 51) (end 119.6 50) (width 0.5) (layer "B.Cu") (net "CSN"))
 (segment (start 113.2 78.8) (end 113.2 78.2) (width 0.5) (layer "B.Cu") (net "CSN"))
 (segment (start 119.6 50) (end 115.6 50) (width 0.5) (layer "B.Cu") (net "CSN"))
 (segment (start 119.6 77.6) (end 120.6 76.6) (width 0.5) (layer "B.Cu") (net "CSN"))
 (segment (start 109 123.2) (end 111.8 126) (width 0.5) (layer "F.Cu") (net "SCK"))
 (segment (start 111.26 54.34) (end 109 56.6) (width 0.5) (layer "F.Cu") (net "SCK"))
 (segment (start 111.8 126) (end 114 126) (width 0.5) (layer "F.Cu") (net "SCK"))
 (segment (start 124.8 126) (end 131.2 126) (width 0.5) (layer "F.Cu") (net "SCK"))
 (segment (start 132.1 126.9) (end 132.1 128.6) (width 0.5) (layer "F.Cu") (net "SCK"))
 (segment (start 131.2 126) (end 132.1 126.9) (width 0.5) (layer "F.Cu") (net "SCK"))
 (segment (start 109 56.6) (end 109 123.2) (width 0.5) (layer "F.Cu") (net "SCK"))
 (via (at 114 126) (size 0.6) (drill 0.3) (layers "F.Cu" "B.Cu") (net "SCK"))
 (via (at 124.8 126) (size 0.6) (drill 0.3) (layers "F.Cu" "B.Cu") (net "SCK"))
 (segment (start 114 126) (end 124.8 126) (width 0.5) (layer "B.Cu") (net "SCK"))
 (segment (start 127.76 130.4) (end 129.56 128.6) (width 0.5) (layer "B.Cu") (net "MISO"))
 (segment (start 108.72 54.34) (end 104.8 58.26) (width 0.5) (layer "B.Cu") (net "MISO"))
 (segment (start 104.8 125.6) (end 109.6 130.4) (width 0.5) (layer "B.Cu") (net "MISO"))
 (segment (start 104.8 58.26) (end 104.8 125.6) (width 0.5) (layer "B.Cu") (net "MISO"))
 (segment (start 109.6 130.4) (end 127.76 130.4) (width 0.5) (layer "B.Cu") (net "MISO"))
 (segment (start 110.4 128.6) (end 116.86 128.6) (width 0.5) (layer "F.Cu") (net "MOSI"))
 (segment (start 106.8 51.881522) (end 106.8 125) (width 0.5) (layer "F.Cu") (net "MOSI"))
 (segment (start 108.181522 50.5) (end 106.8 51.881522) (width 0.5) (layer "F.Cu") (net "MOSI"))
 (segment (start 109.96 50.5) (end 108.181522 50.5) (width 0.5) (layer "F.Cu") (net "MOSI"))
 (segment (start 111.26 51.8) (end 109.96 50.5) (width 0.5) (layer "F.Cu") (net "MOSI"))
 (segment (start 106.8 125) (end 110.4 128.6) (width 0.5) (layer "F.Cu") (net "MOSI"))
 (segment (start 158.6 88.87) (end 159.97 87.5) (width 0.5) (layer "B.Cu") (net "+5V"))
 (segment (start 152.42 103.2) (end 152.42 97.98) (width 0.5) (layer "B.Cu") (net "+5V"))
 (segment (start 158.6 91.8) (end 158.6 88.87) (width 0.5) (layer "B.Cu") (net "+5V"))
 (segment (start 152.42 97.98) (end 158.6 91.8) (width 0.5) (layer "B.Cu") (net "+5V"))
 (segment (start 159.01 54.2) (end 157.6 54.2) (width 0.5) (layer "F.Cu") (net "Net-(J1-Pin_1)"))
 (segment (start 157.6 54.2) (end 153.675 50.275) (width 0.5) (layer "F.Cu") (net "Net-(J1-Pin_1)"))
 (segment (start 159.13 54.08) (end 159.01 54.2) (width 0.5) (layer "F.Cu") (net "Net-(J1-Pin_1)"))
 (segment (start 153.675 50.275) (end 153.675 48.2) (width 0.5) (layer "F.Cu") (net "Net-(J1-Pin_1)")))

